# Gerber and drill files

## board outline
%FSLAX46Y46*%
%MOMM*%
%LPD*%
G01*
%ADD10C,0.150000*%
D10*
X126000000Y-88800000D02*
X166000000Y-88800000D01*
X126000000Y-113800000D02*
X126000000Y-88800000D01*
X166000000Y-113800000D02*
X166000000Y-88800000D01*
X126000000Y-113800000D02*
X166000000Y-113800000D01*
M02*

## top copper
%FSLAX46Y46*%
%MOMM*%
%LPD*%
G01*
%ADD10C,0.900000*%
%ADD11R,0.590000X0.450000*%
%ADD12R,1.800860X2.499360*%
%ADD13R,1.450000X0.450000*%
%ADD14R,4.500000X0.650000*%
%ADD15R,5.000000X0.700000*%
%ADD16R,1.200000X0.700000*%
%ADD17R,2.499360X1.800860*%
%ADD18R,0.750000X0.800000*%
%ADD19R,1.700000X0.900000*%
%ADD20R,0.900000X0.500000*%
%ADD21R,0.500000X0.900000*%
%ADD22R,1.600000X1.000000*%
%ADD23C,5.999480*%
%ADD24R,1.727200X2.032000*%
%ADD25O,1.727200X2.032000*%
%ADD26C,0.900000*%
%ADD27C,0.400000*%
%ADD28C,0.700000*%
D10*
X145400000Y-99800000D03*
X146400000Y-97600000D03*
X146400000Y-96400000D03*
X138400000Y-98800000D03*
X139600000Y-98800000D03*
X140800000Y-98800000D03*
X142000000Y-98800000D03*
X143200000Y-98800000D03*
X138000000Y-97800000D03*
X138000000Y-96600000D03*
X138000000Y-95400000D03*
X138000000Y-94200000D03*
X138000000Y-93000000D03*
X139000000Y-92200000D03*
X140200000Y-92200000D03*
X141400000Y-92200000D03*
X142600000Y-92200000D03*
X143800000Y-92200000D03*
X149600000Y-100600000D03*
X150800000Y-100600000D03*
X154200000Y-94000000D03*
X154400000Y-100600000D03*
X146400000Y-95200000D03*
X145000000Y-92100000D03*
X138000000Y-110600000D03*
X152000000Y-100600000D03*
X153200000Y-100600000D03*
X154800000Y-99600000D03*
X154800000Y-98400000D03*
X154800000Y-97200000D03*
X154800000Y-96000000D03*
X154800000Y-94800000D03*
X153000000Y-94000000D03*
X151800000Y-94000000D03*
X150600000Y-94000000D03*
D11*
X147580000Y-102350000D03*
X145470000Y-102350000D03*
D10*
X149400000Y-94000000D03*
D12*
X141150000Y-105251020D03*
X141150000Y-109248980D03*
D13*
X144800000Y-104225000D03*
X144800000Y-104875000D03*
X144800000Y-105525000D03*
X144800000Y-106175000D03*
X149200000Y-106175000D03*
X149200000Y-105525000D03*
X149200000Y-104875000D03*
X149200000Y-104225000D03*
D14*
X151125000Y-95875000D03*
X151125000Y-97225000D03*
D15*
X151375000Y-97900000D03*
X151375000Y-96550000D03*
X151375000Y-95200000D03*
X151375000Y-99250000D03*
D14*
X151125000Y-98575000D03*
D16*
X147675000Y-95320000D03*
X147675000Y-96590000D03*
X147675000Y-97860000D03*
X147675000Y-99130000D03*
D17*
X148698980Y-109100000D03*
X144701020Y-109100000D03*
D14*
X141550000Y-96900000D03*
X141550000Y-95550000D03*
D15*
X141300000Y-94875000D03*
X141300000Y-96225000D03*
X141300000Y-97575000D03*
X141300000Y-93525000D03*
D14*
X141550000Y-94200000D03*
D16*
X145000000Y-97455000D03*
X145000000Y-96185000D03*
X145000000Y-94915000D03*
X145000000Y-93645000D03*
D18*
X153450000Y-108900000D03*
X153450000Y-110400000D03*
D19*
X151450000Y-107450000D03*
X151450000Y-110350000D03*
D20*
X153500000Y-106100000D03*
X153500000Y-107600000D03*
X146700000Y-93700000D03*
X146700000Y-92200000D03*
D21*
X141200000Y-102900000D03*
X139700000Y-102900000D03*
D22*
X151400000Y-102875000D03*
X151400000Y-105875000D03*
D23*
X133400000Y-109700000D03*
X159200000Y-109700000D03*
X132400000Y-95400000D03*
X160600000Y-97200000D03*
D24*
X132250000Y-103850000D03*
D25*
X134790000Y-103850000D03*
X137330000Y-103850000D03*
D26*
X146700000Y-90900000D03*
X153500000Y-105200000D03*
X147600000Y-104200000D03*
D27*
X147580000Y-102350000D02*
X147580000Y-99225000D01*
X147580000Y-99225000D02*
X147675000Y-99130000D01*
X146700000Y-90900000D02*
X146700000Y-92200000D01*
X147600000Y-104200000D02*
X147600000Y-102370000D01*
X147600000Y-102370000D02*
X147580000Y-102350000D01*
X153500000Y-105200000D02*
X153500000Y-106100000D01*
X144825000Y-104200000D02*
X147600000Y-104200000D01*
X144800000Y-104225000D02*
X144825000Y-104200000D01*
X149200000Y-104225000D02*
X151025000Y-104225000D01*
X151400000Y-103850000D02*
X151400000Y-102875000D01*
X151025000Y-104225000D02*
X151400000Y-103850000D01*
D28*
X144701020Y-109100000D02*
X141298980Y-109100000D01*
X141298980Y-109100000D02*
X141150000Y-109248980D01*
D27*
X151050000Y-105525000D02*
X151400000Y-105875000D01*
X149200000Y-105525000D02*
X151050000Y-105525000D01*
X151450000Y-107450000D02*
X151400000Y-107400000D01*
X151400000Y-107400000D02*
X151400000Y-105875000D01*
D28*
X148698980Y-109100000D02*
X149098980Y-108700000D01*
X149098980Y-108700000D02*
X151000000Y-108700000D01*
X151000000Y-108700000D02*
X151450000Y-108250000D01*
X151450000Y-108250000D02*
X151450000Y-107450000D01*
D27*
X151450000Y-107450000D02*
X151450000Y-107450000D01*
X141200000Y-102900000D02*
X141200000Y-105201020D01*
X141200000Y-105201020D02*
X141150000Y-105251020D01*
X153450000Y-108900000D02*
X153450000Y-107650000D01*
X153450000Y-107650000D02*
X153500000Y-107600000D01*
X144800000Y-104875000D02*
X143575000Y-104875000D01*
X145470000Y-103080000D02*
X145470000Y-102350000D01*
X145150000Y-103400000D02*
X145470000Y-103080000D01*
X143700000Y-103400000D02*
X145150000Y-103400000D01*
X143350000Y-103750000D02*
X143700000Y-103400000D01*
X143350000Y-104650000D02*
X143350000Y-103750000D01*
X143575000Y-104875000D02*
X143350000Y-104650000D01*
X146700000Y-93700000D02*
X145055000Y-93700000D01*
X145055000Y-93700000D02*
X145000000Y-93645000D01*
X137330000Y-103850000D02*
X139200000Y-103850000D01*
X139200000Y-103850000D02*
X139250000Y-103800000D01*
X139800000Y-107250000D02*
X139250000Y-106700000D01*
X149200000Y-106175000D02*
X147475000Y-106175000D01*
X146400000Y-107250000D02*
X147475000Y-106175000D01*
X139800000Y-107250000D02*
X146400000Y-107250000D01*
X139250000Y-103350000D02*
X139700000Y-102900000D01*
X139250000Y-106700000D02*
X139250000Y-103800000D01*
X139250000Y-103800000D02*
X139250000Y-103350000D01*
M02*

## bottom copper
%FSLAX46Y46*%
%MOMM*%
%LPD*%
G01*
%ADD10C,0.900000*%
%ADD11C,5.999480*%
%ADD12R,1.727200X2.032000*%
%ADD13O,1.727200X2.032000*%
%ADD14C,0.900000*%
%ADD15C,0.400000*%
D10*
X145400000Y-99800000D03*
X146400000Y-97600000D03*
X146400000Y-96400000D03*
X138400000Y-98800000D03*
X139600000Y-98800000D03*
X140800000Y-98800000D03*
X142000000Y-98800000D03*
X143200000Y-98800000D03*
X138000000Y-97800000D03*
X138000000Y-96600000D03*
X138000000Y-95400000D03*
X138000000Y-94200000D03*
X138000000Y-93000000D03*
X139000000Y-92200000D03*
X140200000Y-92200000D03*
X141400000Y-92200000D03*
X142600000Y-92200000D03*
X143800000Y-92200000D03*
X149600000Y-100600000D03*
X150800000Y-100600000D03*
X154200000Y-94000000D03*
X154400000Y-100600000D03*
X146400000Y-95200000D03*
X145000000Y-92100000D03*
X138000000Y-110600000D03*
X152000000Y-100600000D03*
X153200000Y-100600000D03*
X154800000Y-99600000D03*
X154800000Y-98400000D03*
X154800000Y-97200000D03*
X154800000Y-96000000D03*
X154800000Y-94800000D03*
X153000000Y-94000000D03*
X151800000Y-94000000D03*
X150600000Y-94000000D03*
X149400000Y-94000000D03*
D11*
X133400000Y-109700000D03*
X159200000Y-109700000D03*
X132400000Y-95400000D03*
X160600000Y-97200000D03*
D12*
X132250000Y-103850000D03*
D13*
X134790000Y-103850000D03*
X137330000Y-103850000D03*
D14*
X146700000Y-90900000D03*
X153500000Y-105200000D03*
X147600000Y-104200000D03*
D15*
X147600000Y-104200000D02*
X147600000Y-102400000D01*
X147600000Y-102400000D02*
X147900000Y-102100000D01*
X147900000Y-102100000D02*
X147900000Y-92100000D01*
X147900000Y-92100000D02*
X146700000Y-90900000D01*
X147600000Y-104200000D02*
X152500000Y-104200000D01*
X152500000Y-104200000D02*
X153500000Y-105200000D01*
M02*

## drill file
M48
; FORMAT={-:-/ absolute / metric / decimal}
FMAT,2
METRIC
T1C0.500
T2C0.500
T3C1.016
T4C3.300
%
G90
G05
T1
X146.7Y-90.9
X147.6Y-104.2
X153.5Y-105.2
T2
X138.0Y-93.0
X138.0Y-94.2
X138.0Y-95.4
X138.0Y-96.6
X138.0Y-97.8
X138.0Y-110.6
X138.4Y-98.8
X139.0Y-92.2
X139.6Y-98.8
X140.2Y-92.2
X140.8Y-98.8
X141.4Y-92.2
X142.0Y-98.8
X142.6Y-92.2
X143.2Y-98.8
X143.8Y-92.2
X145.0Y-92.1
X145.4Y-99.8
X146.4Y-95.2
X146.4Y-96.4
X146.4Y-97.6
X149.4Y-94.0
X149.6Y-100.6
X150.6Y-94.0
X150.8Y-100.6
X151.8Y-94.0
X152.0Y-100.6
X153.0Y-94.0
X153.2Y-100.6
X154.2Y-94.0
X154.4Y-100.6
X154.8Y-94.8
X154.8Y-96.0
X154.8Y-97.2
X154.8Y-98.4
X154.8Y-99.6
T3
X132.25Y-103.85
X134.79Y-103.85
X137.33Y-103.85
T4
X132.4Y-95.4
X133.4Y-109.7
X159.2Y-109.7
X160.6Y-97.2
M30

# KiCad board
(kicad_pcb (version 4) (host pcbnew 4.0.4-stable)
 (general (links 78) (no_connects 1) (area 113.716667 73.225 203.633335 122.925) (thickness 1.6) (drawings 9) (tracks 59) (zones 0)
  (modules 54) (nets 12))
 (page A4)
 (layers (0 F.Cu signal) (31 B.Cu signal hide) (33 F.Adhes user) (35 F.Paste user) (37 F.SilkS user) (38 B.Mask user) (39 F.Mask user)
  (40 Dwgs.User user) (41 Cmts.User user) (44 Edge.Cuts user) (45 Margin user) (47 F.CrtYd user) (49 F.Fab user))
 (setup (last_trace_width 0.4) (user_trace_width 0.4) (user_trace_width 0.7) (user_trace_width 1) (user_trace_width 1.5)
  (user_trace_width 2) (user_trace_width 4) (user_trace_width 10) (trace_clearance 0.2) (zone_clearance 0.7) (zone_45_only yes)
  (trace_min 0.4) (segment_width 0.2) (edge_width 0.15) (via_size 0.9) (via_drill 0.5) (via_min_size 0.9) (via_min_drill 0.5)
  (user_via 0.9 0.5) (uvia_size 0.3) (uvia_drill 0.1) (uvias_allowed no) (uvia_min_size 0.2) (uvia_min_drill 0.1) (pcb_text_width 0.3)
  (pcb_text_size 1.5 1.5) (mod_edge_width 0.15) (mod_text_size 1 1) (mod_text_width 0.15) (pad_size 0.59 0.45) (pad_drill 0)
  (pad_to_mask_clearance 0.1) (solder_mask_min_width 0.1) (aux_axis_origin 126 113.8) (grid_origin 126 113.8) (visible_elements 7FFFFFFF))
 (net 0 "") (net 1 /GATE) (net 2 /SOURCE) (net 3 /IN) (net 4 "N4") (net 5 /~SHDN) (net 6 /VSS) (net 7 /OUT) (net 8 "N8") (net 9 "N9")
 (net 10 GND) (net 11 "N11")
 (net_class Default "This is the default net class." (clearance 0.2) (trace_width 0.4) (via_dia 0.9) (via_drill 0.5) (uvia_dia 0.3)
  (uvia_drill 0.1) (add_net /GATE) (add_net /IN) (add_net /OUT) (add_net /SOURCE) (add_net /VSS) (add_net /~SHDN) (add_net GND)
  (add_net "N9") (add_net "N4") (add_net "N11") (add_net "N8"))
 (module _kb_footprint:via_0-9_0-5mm (layer F.Cu) (at 145.4 99.8)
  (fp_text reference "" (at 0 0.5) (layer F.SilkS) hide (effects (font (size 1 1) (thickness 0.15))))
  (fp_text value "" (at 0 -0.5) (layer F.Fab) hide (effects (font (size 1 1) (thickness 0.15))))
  (pad 1 thru_hole circle (at 0 0) (size 0.9 0.9) (drill 0.5) (layers *.Cu)))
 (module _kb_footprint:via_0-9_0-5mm (layer F.Cu) (at 146.4 97.6)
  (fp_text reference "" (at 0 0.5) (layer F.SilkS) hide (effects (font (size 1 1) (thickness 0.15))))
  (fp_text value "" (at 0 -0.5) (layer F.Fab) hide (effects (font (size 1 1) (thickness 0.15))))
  (pad 1 thru_hole circle (at 0 0) (size 0.9 0.9) (drill 0.5) (layers *.Cu)))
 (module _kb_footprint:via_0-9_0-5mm (layer F.Cu) (at 146.4 96.4)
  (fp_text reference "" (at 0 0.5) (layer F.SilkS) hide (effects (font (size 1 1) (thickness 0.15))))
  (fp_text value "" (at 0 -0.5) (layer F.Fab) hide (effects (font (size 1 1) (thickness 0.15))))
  (pad 1 thru_hole circle (at 0 0) (size 0.9 0.9) (drill 0.5) (layers *.Cu)))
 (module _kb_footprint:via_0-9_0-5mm (layer F.Cu) (at 138.4 98.8)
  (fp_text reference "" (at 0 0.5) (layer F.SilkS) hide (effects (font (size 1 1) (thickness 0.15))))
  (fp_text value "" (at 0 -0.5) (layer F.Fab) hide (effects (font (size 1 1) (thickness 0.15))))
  (pad 1 thru_hole circle (at 0 0) (size 0.9 0.9) (drill 0.5) (layers *.Cu)))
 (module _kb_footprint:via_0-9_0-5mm (layer F.Cu) (at 139.6 98.8)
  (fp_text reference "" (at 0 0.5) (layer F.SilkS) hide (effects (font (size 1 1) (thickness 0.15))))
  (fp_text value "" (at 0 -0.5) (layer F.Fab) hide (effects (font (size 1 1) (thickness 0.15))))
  (pad 1 thru_hole circle (at 0 0) (size 0.9 0.9) (drill 0.5) (layers *.Cu)))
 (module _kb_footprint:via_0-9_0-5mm (layer F.Cu) (at 140.8 98.8)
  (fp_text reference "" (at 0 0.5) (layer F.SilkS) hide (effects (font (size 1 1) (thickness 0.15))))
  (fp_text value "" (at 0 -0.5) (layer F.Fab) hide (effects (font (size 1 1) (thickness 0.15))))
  (pad 1 thru_hole circle (at 0 0) (size 0.9 0.9) (drill 0.5) (layers *.Cu)))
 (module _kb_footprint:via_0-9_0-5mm (layer F.Cu) (at 142 98.8)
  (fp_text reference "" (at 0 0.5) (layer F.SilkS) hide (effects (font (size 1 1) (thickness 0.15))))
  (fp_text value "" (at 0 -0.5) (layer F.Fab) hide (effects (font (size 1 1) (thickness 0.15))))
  (pad 1 thru_hole circle (at 0 0) (size 0.9 0.9) (drill 0.5) (layers *.Cu)))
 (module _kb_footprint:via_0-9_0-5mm (layer F.Cu) (at 143.2 98.8)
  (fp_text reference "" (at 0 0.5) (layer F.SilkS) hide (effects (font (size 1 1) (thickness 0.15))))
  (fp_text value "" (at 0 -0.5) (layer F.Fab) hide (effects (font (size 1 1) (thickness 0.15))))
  (pad 1 thru_hole circle (at 0 0) (size 0.9 0.9) (drill 0.5) (layers *.Cu)))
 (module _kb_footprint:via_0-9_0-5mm (layer F.Cu) (at 138 97.8)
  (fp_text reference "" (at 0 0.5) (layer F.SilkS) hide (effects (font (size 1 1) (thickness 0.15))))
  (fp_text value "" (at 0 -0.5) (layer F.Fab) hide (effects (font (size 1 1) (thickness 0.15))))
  (pad 1 thru_hole circle (at 0 0) (size 0.9 0.9) (drill 0.5) (layers *.Cu)))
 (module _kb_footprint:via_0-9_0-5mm (layer F.Cu) (at 138 96.6)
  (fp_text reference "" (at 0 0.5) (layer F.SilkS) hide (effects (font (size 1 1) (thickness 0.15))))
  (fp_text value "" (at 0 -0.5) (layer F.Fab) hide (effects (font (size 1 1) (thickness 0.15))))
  (pad 1 thru_hole circle (at 0 0) (size 0.9 0.9) (drill 0.5) (layers *.Cu)))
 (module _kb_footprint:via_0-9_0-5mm (layer F.Cu) (at 138 95.4)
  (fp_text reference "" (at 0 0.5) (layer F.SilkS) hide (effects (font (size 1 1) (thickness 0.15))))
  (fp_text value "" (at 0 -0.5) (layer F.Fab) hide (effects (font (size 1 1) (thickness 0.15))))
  (pad 1 thru_hole circle (at 0 0) (size 0.9 0.9) (drill 0.5) (layers *.Cu)))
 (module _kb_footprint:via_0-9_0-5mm (layer F.Cu) (at 138 94.2)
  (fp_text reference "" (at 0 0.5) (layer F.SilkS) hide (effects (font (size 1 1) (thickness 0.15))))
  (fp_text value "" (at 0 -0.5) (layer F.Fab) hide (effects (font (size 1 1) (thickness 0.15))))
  (pad 1 thru_hole circle (at 0 0) (size 0.9 0.9) (drill 0.5) (layers *.Cu)))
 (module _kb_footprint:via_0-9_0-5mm (layer F.Cu) (at 138 93)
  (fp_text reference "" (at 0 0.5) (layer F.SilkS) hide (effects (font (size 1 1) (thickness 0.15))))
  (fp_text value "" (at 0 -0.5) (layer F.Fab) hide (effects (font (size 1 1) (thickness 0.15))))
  (pad 1 thru_hole circle (at 0 0) (size 0.9 0.9) (drill 0.5) (layers *.Cu)))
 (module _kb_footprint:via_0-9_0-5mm (layer F.Cu) (at 139 92.2)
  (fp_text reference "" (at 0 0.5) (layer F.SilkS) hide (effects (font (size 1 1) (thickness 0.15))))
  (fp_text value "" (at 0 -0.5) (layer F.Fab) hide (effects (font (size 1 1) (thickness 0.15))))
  (pad 1 thru_hole circle (at 0 0) (size 0.9 0.9) (drill 0.5) (layers *.Cu)))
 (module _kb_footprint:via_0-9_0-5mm (layer F.Cu) (at 140.2 92.2)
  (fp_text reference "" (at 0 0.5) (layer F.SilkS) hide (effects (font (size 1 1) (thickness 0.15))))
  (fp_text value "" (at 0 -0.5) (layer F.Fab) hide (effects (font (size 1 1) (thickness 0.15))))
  (pad 1 thru_hole circle (at 0 0) (size 0.9 0.9) (drill 0.5) (layers *.Cu)))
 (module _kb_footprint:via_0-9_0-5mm (layer F.Cu) (at 141.4 92.2)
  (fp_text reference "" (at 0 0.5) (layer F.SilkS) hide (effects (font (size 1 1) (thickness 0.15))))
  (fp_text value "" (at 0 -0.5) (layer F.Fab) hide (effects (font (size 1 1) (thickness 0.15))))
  (pad 1 thru_hole circle (at 0 0) (size 0.9 0.9) (drill 0.5) (layers *.Cu)))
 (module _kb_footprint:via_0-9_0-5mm (layer F.Cu) (at 142.6 92.2)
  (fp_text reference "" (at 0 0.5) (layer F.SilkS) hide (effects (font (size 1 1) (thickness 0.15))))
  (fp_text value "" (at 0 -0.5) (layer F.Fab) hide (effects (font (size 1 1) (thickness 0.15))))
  (pad 1 thru_hole circle (at 0 0) (size 0.9 0.9) (drill 0.5) (layers *.Cu)))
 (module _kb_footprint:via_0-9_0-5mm (layer F.Cu) (at 143.8 92.2)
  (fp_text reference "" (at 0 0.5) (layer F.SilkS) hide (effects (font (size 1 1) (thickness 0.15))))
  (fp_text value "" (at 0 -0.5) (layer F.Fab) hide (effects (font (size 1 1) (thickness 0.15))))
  (pad 1 thru_hole circle (at 0 0) (size 0.9 0.9) (drill 0.5) (layers *.Cu)))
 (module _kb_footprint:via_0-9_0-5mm (layer F.Cu) (at 149.6 100.6)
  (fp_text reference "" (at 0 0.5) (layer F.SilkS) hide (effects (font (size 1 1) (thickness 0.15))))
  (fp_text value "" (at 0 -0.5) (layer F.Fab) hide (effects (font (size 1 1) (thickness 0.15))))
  (pad 1 thru_hole circle (at 0 0) (size 0.9 0.9) (drill 0.5) (layers *.Cu)))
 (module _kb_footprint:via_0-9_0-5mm (layer F.Cu) (at 150.8 100.6)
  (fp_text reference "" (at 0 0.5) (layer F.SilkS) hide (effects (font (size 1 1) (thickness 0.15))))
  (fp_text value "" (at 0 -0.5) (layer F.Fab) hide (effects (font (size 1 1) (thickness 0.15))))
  (pad 1 thru_hole circle (at 0 0) (size 0.9 0.9) (drill 0.5) (layers *.Cu)))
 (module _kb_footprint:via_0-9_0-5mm (layer F.Cu) (at 154.2 94)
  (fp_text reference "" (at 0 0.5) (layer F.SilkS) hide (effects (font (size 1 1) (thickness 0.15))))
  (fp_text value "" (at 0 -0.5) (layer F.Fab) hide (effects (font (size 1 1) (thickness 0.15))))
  (pad 1 thru_hole circle (at 0 0) (size 0.9 0.9) (drill 0.5) (layers *.Cu)))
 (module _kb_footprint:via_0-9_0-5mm (layer F.Cu) (at 154.4 100.6)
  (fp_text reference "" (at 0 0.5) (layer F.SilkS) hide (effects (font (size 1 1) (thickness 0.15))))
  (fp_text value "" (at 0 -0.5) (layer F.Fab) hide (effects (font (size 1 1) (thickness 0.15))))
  (pad 1 thru_hole circle (at 0 0) (size 0.9 0.9) (drill 0.5) (layers *.Cu)))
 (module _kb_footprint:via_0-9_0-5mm (layer F.Cu) (at 146.4 95.2)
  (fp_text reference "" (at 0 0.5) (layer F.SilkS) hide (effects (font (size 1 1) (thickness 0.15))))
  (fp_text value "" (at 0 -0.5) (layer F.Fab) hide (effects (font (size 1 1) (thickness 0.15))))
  (pad 1 thru_hole circle (at 0 0) (size 0.9 0.9) (drill 0.5) (layers *.Cu)))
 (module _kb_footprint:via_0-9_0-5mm (layer F.Cu) (at 145 92.1)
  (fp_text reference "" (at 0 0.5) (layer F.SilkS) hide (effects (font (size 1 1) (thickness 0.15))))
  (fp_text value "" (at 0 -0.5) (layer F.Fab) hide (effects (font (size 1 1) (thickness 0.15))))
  (pad 1 thru_hole circle (at 0 0) (size 0.9 0.9) (drill 0.5) (layers *.Cu)))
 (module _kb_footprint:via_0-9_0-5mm (layer F.Cu) (at 138 110.6)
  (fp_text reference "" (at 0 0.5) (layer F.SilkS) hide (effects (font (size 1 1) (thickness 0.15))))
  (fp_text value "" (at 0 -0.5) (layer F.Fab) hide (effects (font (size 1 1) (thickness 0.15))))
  (pad 1 thru_hole circle (at 0 0) (size 0.9 0.9) (drill 0.5) (layers *.Cu)))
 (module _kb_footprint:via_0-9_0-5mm (layer F.Cu) (at 152 100.6)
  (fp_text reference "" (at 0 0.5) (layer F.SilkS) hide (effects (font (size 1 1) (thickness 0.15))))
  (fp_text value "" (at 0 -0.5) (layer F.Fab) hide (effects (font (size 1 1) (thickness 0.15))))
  (pad 1 thru_hole circle (at 0 0) (size 0.9 0.9) (drill 0.5) (layers *.Cu)))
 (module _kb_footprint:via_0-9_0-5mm (layer F.Cu) (at 153.2 100.6)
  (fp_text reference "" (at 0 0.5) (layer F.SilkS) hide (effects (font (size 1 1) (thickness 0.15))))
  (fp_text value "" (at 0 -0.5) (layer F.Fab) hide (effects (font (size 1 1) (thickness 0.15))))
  (pad 1 thru_hole circle (at 0 0) (size 0.9 0.9) (drill 0.5) (layers *.Cu)))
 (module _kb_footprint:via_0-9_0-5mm (layer F.Cu) (at 154.8 99.6)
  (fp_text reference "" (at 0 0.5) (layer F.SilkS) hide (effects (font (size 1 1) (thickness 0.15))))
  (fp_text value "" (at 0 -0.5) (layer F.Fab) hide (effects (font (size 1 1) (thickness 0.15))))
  (pad 1 thru_hole circle (at 0 0) (size 0.9 0.9) (drill 0.5) (layers *.Cu)))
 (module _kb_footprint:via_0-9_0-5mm (layer F.Cu) (at 154.8 98.4)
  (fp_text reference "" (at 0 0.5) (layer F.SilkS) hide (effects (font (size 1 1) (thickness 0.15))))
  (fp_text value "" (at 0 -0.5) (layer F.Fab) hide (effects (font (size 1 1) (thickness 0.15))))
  (pad 1 thru_hole circle (at 0 0) (size 0.9 0.9) (drill 0.5) (layers *.Cu)))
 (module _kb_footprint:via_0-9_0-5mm (layer F.Cu) (at 154.8 97.2)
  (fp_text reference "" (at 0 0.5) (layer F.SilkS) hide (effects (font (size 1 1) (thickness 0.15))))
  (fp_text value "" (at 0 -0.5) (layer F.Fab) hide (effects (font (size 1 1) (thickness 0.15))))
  (pad 1 thru_hole circle (at 0 0) (size 0.9 0.9) (drill 0.5) (layers *.Cu)))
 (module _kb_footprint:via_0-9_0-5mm (layer F.Cu) (at 154.8 96)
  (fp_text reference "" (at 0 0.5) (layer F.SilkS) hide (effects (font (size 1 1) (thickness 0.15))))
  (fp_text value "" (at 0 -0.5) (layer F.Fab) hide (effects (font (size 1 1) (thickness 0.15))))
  (pad 1 thru_hole circle (at 0 0) (size 0.9 0.9) (drill 0.5) (layers *.Cu)))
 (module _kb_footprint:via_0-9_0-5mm (layer F.Cu) (at 154.8 94.8)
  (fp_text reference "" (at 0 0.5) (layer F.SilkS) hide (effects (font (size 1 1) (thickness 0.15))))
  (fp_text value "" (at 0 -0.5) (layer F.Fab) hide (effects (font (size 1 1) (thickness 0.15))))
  (pad 1 thru_hole circle (at 0 0) (size 0.9 0.9) (drill 0.5) (layers *.Cu)))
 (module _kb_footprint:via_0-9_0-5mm (layer F.Cu) (at 153 94)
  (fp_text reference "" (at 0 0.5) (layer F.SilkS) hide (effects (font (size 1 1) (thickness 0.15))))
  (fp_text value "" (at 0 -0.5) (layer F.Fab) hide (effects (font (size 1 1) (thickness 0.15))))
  (pad 1 thru_hole circle (at 0 0) (size 0.9 0.9) (drill 0.5) (layers *.Cu)))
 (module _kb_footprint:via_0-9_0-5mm (layer F.Cu) (at 151.8 94)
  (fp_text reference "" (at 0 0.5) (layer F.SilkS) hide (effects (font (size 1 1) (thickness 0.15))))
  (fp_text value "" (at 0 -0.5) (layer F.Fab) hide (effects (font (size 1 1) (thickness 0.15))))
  (pad 1 thru_hole circle (at 0 0) (size 0.9 0.9) (drill 0.5) (layers *.Cu)))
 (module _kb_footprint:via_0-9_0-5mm (layer F.Cu) (at 150.6 94)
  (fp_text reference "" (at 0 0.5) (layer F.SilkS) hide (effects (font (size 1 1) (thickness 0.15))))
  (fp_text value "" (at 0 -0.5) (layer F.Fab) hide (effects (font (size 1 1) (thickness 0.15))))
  (pad 1 thru_hole circle (at 0 0) (size 0.9 0.9) (drill 0.5) (layers *.Cu)))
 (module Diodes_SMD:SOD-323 (layer F.Cu) (at 146.525 102.35 180)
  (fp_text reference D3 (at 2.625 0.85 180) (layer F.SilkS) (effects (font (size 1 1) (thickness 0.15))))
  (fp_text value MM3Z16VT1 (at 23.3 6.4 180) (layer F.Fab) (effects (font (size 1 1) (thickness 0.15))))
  (pad 1 smd rect (at -1.055 0 180) (size 0.59 0.45) (layers F.Cu F.Paste F.Mask) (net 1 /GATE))
  (pad 2 smd rect (at 1.055 0 180) (size 0.59 0.45) (layers F.Cu F.Paste F.Mask) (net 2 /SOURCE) (zone_connect 1)))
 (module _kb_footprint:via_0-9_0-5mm (layer F.Cu) (at 149.4 94)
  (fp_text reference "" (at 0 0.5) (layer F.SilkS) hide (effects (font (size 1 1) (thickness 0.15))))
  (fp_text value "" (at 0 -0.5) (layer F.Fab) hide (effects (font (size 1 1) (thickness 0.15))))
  (pad 1 thru_hole circle (at 0 0) (size 0.9 0.9) (drill 0.5) (layers *.Cu)))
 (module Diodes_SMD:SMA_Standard (layer F.Cu) (at 141.15 107.25 270)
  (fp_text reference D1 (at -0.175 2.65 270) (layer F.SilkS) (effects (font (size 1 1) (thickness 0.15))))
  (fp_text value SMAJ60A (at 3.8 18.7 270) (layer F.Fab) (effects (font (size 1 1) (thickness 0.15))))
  (pad 1 smd rect (at -1.99898 0 270) (size 2.49936 1.80086) (layers F.Cu F.Paste F.Mask) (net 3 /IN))
  (pad 2 smd rect (at 1.99898 0 270) (size 2.49936 1.80086) (layers F.Cu F.Paste F.Mask) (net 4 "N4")))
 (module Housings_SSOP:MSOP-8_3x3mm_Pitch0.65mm (layer F.Cu) (at 147 105.2)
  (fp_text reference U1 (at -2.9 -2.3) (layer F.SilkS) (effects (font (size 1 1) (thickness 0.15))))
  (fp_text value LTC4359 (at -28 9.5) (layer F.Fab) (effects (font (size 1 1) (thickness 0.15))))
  (pad 1 smd rect (at -2.2 -0.975) (size 1.45 0.45) (layers F.Cu F.Paste F.Mask) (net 1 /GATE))
  (pad 2 smd rect (at -2.2 -0.325) (size 1.45 0.45) (layers F.Cu F.Paste F.Mask) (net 2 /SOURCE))
  (pad 3 smd rect (at -2.2 0.325) (size 1.45 0.45) (layers F.Cu F.Paste F.Mask))
  (pad 4 smd rect (at -2.2 0.975) (size 1.45 0.45) (layers F.Cu F.Paste F.Mask))
  (pad 5 smd rect (at 2.2 0.975) (size 1.45 0.45) (layers F.Cu F.Paste F.Mask) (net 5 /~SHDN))
  (pad 6 smd rect (at 2.2 0.325) (size 1.45 0.45) (layers F.Cu F.Paste F.Mask) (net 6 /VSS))
  (pad 7 smd rect (at 2.2 -0.325) (size 1.45 0.45) (layers F.Cu F.Paste F.Mask))
  (pad 8 smd rect (at 2.2 -0.975) (size 1.45 0.45) (layers F.Cu F.Paste F.Mask) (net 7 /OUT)))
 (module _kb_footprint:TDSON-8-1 (layer F.Cu) (at 150.475 97.225)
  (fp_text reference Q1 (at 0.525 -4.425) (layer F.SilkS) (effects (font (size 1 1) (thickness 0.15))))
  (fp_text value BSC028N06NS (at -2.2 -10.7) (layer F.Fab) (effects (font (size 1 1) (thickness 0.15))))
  (pad 7 smd rect (at 0.65 -1.35) (size 4.5 0.65) (layers F.Cu F.Paste F.Mask))
  (pad 6 smd rect (at 0.65 0) (size 4.5 0.65) (layers F.Cu F.Paste F.Mask))
  (pad 6 smd rect (at 0.9 0.675) (size 5 0.7) (layers F.Cu F.Paste F.Mask))
  (pad 7 smd rect (at 0.9 -0.675) (size 5 0.7) (layers F.Cu F.Paste F.Mask))
  (pad 8 smd rect (at 0.9 -2.025) (size 5 0.7) (layers F.Cu F.Paste F.Mask))
  (pad 5 smd rect (at 0.9 2.025) (size 5 0.7) (layers F.Cu F.Paste F.Mask))
  (pad 5 smd rect (at 0.65 1.35) (size 4.5 0.65) (layers F.Cu F.Paste F.Mask))
  (pad 1 smd rect (at -2.8 -1.905) (size 1.2 0.7) (layers F.Cu F.Paste F.Mask))
  (pad 2 smd rect (at -2.8 -0.635) (size 1.2 0.7) (layers F.Cu F.Paste F.Mask))
  (pad 3 smd rect (at -2.8 0.635) (size 1.2 0.7) (layers F.Cu F.Paste F.Mask))
  (pad 4 smd rect (at -2.8 1.905) (size 1.2 0.7) (layers F.Cu F.Paste F.Mask) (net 1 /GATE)))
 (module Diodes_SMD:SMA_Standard (layer F.Cu) (at 146.7 109.1 180)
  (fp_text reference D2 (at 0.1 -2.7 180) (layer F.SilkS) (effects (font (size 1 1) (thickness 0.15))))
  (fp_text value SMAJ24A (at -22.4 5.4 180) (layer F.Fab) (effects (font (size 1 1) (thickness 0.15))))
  (pad 1 smd rect (at -1.99898 0 180) (size 2.49936 1.80086) (layers F.Cu F.Paste F.Mask) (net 6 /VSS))
  (pad 2 smd rect (at 1.99898 0 180) (size 2.49936 1.80086) (layers F.Cu F.Paste F.Mask) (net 4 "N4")))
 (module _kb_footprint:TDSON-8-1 (layer F.Cu) (at 142.2 95.55 180)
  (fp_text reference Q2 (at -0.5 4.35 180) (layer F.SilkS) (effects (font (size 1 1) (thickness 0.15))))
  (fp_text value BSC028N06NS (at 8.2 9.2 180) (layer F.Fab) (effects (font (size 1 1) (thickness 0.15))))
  (pad 7 smd rect (at 0.65 -1.35 180) (size 4.5 0.65) (layers F.Cu F.Paste F.Mask))
  (pad 6 smd rect (at 0.65 0 180) (size 4.5 0.65) (layers F.Cu F.Paste F.Mask))
  (pad 6 smd rect (at 0.9 0.675 180) (size 5 0.7) (layers F.Cu F.Paste F.Mask))
  (pad 7 smd rect (at 0.9 -0.675 180) (size 5 0.7) (layers F.Cu F.Paste F.Mask))
  (pad 8 smd rect (at 0.9 -2.025 180) (size 5 0.7) (layers F.Cu F.Paste F.Mask))
  (pad 5 smd rect (at 0.9 2.025 180) (size 5 0.7) (layers F.Cu F.Paste F.Mask))
  (pad 5 smd rect (at 0.65 1.35 180) (size 4.5 0.65) (layers F.Cu F.Paste F.Mask))
  (pad 1 smd rect (at -2.8 -1.905 180) (size 1.2 0.7) (layers F.Cu F.Paste F.Mask))
  (pad 2 smd rect (at -2.8 -0.635 180) (size 1.2 0.7) (layers F.Cu F.Paste F.Mask))
  (pad 3 smd rect (at -2.8 0.635 180) (size 1.2 0.7) (layers F.Cu F.Paste F.Mask))
  (pad 4 smd rect (at -2.8 1.905 180) (size 1.2 0.7) (layers F.Cu F.Paste F.Mask) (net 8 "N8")))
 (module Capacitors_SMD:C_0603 (layer F.Cu) (at 153.45 109.65 270)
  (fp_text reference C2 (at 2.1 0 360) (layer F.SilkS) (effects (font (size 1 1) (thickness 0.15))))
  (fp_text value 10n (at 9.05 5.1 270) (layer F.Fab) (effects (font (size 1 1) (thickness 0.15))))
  (pad 1 smd rect (at -0.75 0 270) (size 0.8 0.75) (layers F.Cu F.Paste F.Mask) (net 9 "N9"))
  (pad 2 smd rect (at 0.75 0 270) (size 0.8 0.75) (layers F.Cu F.Paste F.Mask) (zone_connect 1)))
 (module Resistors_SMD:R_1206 (layer F.Cu) (at 151.45 108.9 270)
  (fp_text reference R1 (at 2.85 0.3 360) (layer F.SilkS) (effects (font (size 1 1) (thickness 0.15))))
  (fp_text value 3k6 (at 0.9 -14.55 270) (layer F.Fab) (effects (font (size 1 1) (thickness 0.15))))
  (pad 1 smd rect (at -1.45 0 270) (size 0.9 1.7) (layers F.Cu F.Paste F.Mask) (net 6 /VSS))
  (pad 2 smd rect (at 1.45 0 270) (size 0.9 1.7) (layers F.Cu F.Paste F.Mask) (zone_connect 1)))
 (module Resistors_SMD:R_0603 (layer F.Cu) (at 153.5 106.85 270)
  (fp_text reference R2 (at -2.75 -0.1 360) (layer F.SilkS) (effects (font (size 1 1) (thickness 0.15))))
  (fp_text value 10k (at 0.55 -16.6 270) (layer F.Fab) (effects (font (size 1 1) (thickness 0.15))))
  (pad 1 smd rect (at -0.75 0 270) (size 0.5 0.9) (layers F.Cu F.Paste F.Mask) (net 1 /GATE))
  (pad 2 smd rect (at 0.75 0 270) (size 0.5 0.9) (layers F.Cu F.Paste F.Mask) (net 9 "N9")))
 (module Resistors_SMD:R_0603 (layer F.Cu) (at 146.7 92.95 90)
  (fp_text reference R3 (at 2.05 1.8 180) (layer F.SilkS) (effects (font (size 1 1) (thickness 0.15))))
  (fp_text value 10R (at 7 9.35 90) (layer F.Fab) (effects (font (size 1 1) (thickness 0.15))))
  (pad 1 smd rect (at -0.75 0 90) (size 0.5 0.9) (layers F.Cu F.Paste F.Mask) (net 8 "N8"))
  (pad 2 smd rect (at 0.75 0 90) (size 0.5 0.9) (layers F.Cu F.Paste F.Mask) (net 1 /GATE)))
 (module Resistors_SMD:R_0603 (layer F.Cu) (at 140.45 102.9 180)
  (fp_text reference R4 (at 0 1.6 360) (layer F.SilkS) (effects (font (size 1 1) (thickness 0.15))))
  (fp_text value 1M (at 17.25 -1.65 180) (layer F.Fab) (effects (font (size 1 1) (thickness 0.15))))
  (pad 1 smd rect (at -0.75 0 180) (size 0.5 0.9) (layers F.Cu F.Paste F.Mask) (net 3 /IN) (zone_connect 1))
  (pad 2 smd rect (at 0.75 0 180) (size 0.5 0.9) (layers F.Cu F.Paste F.Mask) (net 5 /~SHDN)))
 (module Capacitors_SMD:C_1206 (layer F.Cu) (at 151.4 104.375 270)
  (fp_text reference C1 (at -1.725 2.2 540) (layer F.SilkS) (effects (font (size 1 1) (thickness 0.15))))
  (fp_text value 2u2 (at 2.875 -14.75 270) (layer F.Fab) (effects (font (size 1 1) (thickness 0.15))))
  (pad 1 smd rect (at -1.5 0 270) (size 1 1.6) (layers F.Cu F.Paste F.Mask) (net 7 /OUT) (zone_connect 1))
  (pad 2 smd rect (at 1.5 0 270) (size 1 1.6) (layers F.Cu F.Paste F.Mask) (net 6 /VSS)))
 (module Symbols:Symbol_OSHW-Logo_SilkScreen (layer F.Cu) (at 174 87)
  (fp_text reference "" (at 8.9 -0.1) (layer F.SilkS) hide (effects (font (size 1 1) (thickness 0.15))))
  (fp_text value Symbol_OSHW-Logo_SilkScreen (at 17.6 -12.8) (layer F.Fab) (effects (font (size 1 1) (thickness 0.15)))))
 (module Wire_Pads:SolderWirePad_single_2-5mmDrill (layer F.Cu) (at 133.4 109.7)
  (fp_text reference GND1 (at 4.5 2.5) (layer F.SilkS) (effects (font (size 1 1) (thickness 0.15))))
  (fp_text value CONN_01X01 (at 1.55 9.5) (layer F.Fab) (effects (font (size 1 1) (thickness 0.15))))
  (pad 1 thru_hole circle (at 0 0) (size 5.99948 5.99948) (drill 3.3) (layers *.Cu *.Mask F.SilkS)))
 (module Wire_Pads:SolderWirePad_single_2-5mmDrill (layer F.Cu) (at 159.2 109.7)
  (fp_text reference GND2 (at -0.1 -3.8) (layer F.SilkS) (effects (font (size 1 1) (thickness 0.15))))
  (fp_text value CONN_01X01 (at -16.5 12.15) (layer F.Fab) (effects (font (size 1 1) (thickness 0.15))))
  (pad 1 thru_hole circle (at 0 0) (size 5.99948 5.99948) (drill 3.3) (layers *.Cu *.Mask F.SilkS)))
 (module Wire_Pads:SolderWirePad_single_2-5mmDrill (layer F.Cu) (at 132.4 95.4)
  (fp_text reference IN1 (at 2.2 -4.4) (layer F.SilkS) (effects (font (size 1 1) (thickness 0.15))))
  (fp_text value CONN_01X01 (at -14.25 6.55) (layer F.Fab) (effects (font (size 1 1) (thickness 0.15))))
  (pad 1 thru_hole circle (at 0 0) (size 5.99948 5.99948) (drill 3.3) (layers *.Cu *.Mask F.SilkS)))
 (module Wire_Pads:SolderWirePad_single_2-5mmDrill (layer F.Cu) (at 160.6 97.2)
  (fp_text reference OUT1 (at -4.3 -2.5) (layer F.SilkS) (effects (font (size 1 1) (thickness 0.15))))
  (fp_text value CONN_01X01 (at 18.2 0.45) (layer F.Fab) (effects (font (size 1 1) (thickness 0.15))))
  (pad 1 thru_hole circle (at 0 0) (size 5.99948 5.99948) (drill 3.3) (layers *.Cu *.Mask F.SilkS)))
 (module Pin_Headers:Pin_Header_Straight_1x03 (layer F.Cu) (at 132.25 103.85 90)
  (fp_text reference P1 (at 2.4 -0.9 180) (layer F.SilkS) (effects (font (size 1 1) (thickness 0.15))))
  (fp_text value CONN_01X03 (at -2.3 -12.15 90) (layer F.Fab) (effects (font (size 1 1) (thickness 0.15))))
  (pad 1 thru_hole rect (at 0 0 90) (size 2.032 1.7272) (drill 1.016) (layers *.Cu *.Mask F.SilkS))
  (pad 2 thru_hole oval (at 0 2.54 90) (size 2.032 1.7272) (drill 1.016) (layers *.Cu *.Mask F.SilkS))
  (pad 3 thru_hole oval (at 0 5.08 90) (size 2.032 1.7272) (drill 1.016) (layers *.Cu *.Mask F.SilkS) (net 5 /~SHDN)))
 (gr_line (start 126 88.8) (end 166 88.8) (angle 90) (layer Edge.Cuts) (width 0.15))
 (gr_line (start 126 113.8) (end 126 88.8) (angle 90) (layer Edge.Cuts) (width 0.15))
 (gr_line (start 166 113.8) (end 166 88.8) (angle 90) (layer Edge.Cuts) (width 0.15))
 (gr_line (start 126 113.8) (end 166 113.8) (angle 90) (layer Edge.Cuts) (width 0.15))
 (segment (start 147.58 102.35) (end 147.58 99.225) (width 0.4) (layer F.Cu) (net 1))
 (segment (start 147.58 99.225) (end 147.675 99.13) (width 0.4) (layer F.Cu) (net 1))
 (segment (start 147.6 104.2) (end 147.6 102.4) (width 0.4) (layer B.Cu) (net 1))
 (segment (start 147.6 102.4) (end 147.9 102.1) (width 0.4) (layer B.Cu) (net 1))
 (segment (start 147.9 102.1) (end 147.9 92.1) (width 0.4) (layer B.Cu) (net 1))
 (segment (start 147.9 92.1) (end 146.7 90.9) (width 0.4) (layer B.Cu) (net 1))
 (segment (start 146.7 90.9) (end 146.7 92.2) (width 0.4) (layer F.Cu) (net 1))
 (segment (start 147.6 104.2) (end 147.6 102.37) (width 0.4) (layer F.Cu) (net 1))
 (segment (start 147.6 102.37) (end 147.58 102.35) (width 0.4) (layer F.Cu) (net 1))
 (segment (start 147.6 104.2) (end 152.5 104.2) (width 0.4) (layer B.Cu) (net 1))
 (segment (start 153.5 105.2) (end 153.5 106.1) (width 0.4) (layer F.Cu) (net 1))
 (segment (start 152.5 104.2) (end 153.5 105.2) (width 0.4) (layer B.Cu) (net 1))
 (segment (start 144.825 104.2) (end 147.6 104.2) (width 0.4) (layer F.Cu) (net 1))
 (segment (start 144.8 104.225) (end 144.825 104.2) (width 0.4) (layer F.Cu) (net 1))
 (segment (start 149.2 104.225) (end 151.025 104.225) (width 0.4) (layer F.Cu) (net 7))
 (segment (start 151.4 103.85) (end 151.4 102.875) (width 0.4) (layer F.Cu) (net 7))
 (segment (start 151.025 104.225) (end 151.4 103.85) (width 0.4) (layer F.Cu) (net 7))
 (segment (start 144.70102 109.1) (end 141.29898 109.1) (width 0.7) (layer F.Cu) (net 4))
 (segment (start 141.29898 109.1) (end 141.15 109.24898) (width 0.7) (layer F.Cu) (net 4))
 (segment (start 151.05 105.525) (end 151.4 105.875) (width 0.4) (layer F.Cu) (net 6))
 (segment (start 149.2 105.525) (end 151.05 105.525) (width 0.4) (layer F.Cu) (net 6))
 (segment (start 151.45 107.45) (end 151.4 107.4) (width 0.4) (layer F.Cu) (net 6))
 (segment (start 151.4 107.4) (end 151.4 105.875) (width 0.4) (layer F.Cu) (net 6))
 (segment (start 148.69898 109.1) (end 149.09898 108.7) (width 0.7) (layer F.Cu) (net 6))
 (segment (start 149.09898 108.7) (end 151 108.7) (width 0.7) (layer F.Cu) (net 6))
 (segment (start 151 108.7) (end 151.45 108.25) (width 0.7) (layer F.Cu) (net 6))
 (segment (start 151.45 108.25) (end 151.45 107.45) (width 0.7) (layer F.Cu) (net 6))
 (segment (start 151.45 107.45) (end 151.45 107.45) (width 0.4) (layer F.Cu) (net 6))
 (segment (start 141.2 102.9) (end 141.2 105.20102) (width 0.4) (layer F.Cu) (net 3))
 (segment (start 141.2 105.20102) (end 141.15 105.25102) (width 0.4) (layer F.Cu) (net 3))
 (segment (start 153.45 108.9) (end 153.45 107.65) (width 0.4) (layer F.Cu) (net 9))
 (segment (start 153.45 107.65) (end 153.5 107.6) (width 0.4) (layer F.Cu) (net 9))
 (segment (start 144.8 104.875) (end 143.575 104.875) (width 0.4) (layer F.Cu) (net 2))
 (segment (start 145.47 103.08) (end 145.47 102.35) (width 0.4) (layer F.Cu) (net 2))
 (segment (start 145.15 103.4) (end 145.47 103.08) (width 0.4) (layer F.Cu) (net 2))
 (segment (start 143.7 103.4) (end 145.15 103.4) (width 0.4) (layer F.Cu) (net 2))
 (segment (start 143.35 103.75) (end 143.7 103.4) (width 0.4) (layer F.Cu) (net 2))
 (segment (start 143.35 104.65) (end 143.35 103.75) (width 0.4) (layer F.Cu) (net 2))
 (segment (start 143.575 104.875) (end 143.35 104.65) (width 0.4) (layer F.Cu) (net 2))
 (segment (start 146.7 93.7) (end 145.055 93.7) (width 0.4) (layer F.Cu) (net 8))
 (segment (start 145.055 93.7) (end 145 93.645) (width 0.4) (layer F.Cu) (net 8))
 (segment (start 137.33 103.85) (end 139.2 103.85) (width 0.4) (layer F.Cu) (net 5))
 (segment (start 139.2 103.85) (end 139.25 103.8) (width 0.4) (layer F.Cu) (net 5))
 (segment (start 139.8 107.25) (end 139.25 106.7) (width 0.4) (layer F.Cu) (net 5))
 (segment (start 149.2 106.175) (end 147.475 106.175) (width 0.4) (layer F.Cu) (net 5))
 (segment (start 146.4 107.25) (end 147.475 106.175) (width 0.4) (layer F.Cu) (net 5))
 (segment (start 139.8 107.25) (end 146.4 107.25) (width 0.4) (layer F.Cu) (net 5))
 (segment (start 139.25 103.35) (end 139.7 102.9) (width 0.4) (layer F.Cu) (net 5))
 (segment (start 139.25 106.7) (end 139.25 103.8) (width 0.4) (layer F.Cu) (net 5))
 (segment (start 139.25 103.8) (end 139.25 103.35) (width 0.4) (layer F.Cu) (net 5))
 (via (at 146.7 90.9) (size 0.9) (layers F.Cu B.Cu) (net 1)) (via (at 153.5 105.2) (size 0.9) (layers F.Cu B.Cu) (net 1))
 (via (at 147.6 104.2) (size 0.9) (layers F.Cu B.Cu) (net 1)))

